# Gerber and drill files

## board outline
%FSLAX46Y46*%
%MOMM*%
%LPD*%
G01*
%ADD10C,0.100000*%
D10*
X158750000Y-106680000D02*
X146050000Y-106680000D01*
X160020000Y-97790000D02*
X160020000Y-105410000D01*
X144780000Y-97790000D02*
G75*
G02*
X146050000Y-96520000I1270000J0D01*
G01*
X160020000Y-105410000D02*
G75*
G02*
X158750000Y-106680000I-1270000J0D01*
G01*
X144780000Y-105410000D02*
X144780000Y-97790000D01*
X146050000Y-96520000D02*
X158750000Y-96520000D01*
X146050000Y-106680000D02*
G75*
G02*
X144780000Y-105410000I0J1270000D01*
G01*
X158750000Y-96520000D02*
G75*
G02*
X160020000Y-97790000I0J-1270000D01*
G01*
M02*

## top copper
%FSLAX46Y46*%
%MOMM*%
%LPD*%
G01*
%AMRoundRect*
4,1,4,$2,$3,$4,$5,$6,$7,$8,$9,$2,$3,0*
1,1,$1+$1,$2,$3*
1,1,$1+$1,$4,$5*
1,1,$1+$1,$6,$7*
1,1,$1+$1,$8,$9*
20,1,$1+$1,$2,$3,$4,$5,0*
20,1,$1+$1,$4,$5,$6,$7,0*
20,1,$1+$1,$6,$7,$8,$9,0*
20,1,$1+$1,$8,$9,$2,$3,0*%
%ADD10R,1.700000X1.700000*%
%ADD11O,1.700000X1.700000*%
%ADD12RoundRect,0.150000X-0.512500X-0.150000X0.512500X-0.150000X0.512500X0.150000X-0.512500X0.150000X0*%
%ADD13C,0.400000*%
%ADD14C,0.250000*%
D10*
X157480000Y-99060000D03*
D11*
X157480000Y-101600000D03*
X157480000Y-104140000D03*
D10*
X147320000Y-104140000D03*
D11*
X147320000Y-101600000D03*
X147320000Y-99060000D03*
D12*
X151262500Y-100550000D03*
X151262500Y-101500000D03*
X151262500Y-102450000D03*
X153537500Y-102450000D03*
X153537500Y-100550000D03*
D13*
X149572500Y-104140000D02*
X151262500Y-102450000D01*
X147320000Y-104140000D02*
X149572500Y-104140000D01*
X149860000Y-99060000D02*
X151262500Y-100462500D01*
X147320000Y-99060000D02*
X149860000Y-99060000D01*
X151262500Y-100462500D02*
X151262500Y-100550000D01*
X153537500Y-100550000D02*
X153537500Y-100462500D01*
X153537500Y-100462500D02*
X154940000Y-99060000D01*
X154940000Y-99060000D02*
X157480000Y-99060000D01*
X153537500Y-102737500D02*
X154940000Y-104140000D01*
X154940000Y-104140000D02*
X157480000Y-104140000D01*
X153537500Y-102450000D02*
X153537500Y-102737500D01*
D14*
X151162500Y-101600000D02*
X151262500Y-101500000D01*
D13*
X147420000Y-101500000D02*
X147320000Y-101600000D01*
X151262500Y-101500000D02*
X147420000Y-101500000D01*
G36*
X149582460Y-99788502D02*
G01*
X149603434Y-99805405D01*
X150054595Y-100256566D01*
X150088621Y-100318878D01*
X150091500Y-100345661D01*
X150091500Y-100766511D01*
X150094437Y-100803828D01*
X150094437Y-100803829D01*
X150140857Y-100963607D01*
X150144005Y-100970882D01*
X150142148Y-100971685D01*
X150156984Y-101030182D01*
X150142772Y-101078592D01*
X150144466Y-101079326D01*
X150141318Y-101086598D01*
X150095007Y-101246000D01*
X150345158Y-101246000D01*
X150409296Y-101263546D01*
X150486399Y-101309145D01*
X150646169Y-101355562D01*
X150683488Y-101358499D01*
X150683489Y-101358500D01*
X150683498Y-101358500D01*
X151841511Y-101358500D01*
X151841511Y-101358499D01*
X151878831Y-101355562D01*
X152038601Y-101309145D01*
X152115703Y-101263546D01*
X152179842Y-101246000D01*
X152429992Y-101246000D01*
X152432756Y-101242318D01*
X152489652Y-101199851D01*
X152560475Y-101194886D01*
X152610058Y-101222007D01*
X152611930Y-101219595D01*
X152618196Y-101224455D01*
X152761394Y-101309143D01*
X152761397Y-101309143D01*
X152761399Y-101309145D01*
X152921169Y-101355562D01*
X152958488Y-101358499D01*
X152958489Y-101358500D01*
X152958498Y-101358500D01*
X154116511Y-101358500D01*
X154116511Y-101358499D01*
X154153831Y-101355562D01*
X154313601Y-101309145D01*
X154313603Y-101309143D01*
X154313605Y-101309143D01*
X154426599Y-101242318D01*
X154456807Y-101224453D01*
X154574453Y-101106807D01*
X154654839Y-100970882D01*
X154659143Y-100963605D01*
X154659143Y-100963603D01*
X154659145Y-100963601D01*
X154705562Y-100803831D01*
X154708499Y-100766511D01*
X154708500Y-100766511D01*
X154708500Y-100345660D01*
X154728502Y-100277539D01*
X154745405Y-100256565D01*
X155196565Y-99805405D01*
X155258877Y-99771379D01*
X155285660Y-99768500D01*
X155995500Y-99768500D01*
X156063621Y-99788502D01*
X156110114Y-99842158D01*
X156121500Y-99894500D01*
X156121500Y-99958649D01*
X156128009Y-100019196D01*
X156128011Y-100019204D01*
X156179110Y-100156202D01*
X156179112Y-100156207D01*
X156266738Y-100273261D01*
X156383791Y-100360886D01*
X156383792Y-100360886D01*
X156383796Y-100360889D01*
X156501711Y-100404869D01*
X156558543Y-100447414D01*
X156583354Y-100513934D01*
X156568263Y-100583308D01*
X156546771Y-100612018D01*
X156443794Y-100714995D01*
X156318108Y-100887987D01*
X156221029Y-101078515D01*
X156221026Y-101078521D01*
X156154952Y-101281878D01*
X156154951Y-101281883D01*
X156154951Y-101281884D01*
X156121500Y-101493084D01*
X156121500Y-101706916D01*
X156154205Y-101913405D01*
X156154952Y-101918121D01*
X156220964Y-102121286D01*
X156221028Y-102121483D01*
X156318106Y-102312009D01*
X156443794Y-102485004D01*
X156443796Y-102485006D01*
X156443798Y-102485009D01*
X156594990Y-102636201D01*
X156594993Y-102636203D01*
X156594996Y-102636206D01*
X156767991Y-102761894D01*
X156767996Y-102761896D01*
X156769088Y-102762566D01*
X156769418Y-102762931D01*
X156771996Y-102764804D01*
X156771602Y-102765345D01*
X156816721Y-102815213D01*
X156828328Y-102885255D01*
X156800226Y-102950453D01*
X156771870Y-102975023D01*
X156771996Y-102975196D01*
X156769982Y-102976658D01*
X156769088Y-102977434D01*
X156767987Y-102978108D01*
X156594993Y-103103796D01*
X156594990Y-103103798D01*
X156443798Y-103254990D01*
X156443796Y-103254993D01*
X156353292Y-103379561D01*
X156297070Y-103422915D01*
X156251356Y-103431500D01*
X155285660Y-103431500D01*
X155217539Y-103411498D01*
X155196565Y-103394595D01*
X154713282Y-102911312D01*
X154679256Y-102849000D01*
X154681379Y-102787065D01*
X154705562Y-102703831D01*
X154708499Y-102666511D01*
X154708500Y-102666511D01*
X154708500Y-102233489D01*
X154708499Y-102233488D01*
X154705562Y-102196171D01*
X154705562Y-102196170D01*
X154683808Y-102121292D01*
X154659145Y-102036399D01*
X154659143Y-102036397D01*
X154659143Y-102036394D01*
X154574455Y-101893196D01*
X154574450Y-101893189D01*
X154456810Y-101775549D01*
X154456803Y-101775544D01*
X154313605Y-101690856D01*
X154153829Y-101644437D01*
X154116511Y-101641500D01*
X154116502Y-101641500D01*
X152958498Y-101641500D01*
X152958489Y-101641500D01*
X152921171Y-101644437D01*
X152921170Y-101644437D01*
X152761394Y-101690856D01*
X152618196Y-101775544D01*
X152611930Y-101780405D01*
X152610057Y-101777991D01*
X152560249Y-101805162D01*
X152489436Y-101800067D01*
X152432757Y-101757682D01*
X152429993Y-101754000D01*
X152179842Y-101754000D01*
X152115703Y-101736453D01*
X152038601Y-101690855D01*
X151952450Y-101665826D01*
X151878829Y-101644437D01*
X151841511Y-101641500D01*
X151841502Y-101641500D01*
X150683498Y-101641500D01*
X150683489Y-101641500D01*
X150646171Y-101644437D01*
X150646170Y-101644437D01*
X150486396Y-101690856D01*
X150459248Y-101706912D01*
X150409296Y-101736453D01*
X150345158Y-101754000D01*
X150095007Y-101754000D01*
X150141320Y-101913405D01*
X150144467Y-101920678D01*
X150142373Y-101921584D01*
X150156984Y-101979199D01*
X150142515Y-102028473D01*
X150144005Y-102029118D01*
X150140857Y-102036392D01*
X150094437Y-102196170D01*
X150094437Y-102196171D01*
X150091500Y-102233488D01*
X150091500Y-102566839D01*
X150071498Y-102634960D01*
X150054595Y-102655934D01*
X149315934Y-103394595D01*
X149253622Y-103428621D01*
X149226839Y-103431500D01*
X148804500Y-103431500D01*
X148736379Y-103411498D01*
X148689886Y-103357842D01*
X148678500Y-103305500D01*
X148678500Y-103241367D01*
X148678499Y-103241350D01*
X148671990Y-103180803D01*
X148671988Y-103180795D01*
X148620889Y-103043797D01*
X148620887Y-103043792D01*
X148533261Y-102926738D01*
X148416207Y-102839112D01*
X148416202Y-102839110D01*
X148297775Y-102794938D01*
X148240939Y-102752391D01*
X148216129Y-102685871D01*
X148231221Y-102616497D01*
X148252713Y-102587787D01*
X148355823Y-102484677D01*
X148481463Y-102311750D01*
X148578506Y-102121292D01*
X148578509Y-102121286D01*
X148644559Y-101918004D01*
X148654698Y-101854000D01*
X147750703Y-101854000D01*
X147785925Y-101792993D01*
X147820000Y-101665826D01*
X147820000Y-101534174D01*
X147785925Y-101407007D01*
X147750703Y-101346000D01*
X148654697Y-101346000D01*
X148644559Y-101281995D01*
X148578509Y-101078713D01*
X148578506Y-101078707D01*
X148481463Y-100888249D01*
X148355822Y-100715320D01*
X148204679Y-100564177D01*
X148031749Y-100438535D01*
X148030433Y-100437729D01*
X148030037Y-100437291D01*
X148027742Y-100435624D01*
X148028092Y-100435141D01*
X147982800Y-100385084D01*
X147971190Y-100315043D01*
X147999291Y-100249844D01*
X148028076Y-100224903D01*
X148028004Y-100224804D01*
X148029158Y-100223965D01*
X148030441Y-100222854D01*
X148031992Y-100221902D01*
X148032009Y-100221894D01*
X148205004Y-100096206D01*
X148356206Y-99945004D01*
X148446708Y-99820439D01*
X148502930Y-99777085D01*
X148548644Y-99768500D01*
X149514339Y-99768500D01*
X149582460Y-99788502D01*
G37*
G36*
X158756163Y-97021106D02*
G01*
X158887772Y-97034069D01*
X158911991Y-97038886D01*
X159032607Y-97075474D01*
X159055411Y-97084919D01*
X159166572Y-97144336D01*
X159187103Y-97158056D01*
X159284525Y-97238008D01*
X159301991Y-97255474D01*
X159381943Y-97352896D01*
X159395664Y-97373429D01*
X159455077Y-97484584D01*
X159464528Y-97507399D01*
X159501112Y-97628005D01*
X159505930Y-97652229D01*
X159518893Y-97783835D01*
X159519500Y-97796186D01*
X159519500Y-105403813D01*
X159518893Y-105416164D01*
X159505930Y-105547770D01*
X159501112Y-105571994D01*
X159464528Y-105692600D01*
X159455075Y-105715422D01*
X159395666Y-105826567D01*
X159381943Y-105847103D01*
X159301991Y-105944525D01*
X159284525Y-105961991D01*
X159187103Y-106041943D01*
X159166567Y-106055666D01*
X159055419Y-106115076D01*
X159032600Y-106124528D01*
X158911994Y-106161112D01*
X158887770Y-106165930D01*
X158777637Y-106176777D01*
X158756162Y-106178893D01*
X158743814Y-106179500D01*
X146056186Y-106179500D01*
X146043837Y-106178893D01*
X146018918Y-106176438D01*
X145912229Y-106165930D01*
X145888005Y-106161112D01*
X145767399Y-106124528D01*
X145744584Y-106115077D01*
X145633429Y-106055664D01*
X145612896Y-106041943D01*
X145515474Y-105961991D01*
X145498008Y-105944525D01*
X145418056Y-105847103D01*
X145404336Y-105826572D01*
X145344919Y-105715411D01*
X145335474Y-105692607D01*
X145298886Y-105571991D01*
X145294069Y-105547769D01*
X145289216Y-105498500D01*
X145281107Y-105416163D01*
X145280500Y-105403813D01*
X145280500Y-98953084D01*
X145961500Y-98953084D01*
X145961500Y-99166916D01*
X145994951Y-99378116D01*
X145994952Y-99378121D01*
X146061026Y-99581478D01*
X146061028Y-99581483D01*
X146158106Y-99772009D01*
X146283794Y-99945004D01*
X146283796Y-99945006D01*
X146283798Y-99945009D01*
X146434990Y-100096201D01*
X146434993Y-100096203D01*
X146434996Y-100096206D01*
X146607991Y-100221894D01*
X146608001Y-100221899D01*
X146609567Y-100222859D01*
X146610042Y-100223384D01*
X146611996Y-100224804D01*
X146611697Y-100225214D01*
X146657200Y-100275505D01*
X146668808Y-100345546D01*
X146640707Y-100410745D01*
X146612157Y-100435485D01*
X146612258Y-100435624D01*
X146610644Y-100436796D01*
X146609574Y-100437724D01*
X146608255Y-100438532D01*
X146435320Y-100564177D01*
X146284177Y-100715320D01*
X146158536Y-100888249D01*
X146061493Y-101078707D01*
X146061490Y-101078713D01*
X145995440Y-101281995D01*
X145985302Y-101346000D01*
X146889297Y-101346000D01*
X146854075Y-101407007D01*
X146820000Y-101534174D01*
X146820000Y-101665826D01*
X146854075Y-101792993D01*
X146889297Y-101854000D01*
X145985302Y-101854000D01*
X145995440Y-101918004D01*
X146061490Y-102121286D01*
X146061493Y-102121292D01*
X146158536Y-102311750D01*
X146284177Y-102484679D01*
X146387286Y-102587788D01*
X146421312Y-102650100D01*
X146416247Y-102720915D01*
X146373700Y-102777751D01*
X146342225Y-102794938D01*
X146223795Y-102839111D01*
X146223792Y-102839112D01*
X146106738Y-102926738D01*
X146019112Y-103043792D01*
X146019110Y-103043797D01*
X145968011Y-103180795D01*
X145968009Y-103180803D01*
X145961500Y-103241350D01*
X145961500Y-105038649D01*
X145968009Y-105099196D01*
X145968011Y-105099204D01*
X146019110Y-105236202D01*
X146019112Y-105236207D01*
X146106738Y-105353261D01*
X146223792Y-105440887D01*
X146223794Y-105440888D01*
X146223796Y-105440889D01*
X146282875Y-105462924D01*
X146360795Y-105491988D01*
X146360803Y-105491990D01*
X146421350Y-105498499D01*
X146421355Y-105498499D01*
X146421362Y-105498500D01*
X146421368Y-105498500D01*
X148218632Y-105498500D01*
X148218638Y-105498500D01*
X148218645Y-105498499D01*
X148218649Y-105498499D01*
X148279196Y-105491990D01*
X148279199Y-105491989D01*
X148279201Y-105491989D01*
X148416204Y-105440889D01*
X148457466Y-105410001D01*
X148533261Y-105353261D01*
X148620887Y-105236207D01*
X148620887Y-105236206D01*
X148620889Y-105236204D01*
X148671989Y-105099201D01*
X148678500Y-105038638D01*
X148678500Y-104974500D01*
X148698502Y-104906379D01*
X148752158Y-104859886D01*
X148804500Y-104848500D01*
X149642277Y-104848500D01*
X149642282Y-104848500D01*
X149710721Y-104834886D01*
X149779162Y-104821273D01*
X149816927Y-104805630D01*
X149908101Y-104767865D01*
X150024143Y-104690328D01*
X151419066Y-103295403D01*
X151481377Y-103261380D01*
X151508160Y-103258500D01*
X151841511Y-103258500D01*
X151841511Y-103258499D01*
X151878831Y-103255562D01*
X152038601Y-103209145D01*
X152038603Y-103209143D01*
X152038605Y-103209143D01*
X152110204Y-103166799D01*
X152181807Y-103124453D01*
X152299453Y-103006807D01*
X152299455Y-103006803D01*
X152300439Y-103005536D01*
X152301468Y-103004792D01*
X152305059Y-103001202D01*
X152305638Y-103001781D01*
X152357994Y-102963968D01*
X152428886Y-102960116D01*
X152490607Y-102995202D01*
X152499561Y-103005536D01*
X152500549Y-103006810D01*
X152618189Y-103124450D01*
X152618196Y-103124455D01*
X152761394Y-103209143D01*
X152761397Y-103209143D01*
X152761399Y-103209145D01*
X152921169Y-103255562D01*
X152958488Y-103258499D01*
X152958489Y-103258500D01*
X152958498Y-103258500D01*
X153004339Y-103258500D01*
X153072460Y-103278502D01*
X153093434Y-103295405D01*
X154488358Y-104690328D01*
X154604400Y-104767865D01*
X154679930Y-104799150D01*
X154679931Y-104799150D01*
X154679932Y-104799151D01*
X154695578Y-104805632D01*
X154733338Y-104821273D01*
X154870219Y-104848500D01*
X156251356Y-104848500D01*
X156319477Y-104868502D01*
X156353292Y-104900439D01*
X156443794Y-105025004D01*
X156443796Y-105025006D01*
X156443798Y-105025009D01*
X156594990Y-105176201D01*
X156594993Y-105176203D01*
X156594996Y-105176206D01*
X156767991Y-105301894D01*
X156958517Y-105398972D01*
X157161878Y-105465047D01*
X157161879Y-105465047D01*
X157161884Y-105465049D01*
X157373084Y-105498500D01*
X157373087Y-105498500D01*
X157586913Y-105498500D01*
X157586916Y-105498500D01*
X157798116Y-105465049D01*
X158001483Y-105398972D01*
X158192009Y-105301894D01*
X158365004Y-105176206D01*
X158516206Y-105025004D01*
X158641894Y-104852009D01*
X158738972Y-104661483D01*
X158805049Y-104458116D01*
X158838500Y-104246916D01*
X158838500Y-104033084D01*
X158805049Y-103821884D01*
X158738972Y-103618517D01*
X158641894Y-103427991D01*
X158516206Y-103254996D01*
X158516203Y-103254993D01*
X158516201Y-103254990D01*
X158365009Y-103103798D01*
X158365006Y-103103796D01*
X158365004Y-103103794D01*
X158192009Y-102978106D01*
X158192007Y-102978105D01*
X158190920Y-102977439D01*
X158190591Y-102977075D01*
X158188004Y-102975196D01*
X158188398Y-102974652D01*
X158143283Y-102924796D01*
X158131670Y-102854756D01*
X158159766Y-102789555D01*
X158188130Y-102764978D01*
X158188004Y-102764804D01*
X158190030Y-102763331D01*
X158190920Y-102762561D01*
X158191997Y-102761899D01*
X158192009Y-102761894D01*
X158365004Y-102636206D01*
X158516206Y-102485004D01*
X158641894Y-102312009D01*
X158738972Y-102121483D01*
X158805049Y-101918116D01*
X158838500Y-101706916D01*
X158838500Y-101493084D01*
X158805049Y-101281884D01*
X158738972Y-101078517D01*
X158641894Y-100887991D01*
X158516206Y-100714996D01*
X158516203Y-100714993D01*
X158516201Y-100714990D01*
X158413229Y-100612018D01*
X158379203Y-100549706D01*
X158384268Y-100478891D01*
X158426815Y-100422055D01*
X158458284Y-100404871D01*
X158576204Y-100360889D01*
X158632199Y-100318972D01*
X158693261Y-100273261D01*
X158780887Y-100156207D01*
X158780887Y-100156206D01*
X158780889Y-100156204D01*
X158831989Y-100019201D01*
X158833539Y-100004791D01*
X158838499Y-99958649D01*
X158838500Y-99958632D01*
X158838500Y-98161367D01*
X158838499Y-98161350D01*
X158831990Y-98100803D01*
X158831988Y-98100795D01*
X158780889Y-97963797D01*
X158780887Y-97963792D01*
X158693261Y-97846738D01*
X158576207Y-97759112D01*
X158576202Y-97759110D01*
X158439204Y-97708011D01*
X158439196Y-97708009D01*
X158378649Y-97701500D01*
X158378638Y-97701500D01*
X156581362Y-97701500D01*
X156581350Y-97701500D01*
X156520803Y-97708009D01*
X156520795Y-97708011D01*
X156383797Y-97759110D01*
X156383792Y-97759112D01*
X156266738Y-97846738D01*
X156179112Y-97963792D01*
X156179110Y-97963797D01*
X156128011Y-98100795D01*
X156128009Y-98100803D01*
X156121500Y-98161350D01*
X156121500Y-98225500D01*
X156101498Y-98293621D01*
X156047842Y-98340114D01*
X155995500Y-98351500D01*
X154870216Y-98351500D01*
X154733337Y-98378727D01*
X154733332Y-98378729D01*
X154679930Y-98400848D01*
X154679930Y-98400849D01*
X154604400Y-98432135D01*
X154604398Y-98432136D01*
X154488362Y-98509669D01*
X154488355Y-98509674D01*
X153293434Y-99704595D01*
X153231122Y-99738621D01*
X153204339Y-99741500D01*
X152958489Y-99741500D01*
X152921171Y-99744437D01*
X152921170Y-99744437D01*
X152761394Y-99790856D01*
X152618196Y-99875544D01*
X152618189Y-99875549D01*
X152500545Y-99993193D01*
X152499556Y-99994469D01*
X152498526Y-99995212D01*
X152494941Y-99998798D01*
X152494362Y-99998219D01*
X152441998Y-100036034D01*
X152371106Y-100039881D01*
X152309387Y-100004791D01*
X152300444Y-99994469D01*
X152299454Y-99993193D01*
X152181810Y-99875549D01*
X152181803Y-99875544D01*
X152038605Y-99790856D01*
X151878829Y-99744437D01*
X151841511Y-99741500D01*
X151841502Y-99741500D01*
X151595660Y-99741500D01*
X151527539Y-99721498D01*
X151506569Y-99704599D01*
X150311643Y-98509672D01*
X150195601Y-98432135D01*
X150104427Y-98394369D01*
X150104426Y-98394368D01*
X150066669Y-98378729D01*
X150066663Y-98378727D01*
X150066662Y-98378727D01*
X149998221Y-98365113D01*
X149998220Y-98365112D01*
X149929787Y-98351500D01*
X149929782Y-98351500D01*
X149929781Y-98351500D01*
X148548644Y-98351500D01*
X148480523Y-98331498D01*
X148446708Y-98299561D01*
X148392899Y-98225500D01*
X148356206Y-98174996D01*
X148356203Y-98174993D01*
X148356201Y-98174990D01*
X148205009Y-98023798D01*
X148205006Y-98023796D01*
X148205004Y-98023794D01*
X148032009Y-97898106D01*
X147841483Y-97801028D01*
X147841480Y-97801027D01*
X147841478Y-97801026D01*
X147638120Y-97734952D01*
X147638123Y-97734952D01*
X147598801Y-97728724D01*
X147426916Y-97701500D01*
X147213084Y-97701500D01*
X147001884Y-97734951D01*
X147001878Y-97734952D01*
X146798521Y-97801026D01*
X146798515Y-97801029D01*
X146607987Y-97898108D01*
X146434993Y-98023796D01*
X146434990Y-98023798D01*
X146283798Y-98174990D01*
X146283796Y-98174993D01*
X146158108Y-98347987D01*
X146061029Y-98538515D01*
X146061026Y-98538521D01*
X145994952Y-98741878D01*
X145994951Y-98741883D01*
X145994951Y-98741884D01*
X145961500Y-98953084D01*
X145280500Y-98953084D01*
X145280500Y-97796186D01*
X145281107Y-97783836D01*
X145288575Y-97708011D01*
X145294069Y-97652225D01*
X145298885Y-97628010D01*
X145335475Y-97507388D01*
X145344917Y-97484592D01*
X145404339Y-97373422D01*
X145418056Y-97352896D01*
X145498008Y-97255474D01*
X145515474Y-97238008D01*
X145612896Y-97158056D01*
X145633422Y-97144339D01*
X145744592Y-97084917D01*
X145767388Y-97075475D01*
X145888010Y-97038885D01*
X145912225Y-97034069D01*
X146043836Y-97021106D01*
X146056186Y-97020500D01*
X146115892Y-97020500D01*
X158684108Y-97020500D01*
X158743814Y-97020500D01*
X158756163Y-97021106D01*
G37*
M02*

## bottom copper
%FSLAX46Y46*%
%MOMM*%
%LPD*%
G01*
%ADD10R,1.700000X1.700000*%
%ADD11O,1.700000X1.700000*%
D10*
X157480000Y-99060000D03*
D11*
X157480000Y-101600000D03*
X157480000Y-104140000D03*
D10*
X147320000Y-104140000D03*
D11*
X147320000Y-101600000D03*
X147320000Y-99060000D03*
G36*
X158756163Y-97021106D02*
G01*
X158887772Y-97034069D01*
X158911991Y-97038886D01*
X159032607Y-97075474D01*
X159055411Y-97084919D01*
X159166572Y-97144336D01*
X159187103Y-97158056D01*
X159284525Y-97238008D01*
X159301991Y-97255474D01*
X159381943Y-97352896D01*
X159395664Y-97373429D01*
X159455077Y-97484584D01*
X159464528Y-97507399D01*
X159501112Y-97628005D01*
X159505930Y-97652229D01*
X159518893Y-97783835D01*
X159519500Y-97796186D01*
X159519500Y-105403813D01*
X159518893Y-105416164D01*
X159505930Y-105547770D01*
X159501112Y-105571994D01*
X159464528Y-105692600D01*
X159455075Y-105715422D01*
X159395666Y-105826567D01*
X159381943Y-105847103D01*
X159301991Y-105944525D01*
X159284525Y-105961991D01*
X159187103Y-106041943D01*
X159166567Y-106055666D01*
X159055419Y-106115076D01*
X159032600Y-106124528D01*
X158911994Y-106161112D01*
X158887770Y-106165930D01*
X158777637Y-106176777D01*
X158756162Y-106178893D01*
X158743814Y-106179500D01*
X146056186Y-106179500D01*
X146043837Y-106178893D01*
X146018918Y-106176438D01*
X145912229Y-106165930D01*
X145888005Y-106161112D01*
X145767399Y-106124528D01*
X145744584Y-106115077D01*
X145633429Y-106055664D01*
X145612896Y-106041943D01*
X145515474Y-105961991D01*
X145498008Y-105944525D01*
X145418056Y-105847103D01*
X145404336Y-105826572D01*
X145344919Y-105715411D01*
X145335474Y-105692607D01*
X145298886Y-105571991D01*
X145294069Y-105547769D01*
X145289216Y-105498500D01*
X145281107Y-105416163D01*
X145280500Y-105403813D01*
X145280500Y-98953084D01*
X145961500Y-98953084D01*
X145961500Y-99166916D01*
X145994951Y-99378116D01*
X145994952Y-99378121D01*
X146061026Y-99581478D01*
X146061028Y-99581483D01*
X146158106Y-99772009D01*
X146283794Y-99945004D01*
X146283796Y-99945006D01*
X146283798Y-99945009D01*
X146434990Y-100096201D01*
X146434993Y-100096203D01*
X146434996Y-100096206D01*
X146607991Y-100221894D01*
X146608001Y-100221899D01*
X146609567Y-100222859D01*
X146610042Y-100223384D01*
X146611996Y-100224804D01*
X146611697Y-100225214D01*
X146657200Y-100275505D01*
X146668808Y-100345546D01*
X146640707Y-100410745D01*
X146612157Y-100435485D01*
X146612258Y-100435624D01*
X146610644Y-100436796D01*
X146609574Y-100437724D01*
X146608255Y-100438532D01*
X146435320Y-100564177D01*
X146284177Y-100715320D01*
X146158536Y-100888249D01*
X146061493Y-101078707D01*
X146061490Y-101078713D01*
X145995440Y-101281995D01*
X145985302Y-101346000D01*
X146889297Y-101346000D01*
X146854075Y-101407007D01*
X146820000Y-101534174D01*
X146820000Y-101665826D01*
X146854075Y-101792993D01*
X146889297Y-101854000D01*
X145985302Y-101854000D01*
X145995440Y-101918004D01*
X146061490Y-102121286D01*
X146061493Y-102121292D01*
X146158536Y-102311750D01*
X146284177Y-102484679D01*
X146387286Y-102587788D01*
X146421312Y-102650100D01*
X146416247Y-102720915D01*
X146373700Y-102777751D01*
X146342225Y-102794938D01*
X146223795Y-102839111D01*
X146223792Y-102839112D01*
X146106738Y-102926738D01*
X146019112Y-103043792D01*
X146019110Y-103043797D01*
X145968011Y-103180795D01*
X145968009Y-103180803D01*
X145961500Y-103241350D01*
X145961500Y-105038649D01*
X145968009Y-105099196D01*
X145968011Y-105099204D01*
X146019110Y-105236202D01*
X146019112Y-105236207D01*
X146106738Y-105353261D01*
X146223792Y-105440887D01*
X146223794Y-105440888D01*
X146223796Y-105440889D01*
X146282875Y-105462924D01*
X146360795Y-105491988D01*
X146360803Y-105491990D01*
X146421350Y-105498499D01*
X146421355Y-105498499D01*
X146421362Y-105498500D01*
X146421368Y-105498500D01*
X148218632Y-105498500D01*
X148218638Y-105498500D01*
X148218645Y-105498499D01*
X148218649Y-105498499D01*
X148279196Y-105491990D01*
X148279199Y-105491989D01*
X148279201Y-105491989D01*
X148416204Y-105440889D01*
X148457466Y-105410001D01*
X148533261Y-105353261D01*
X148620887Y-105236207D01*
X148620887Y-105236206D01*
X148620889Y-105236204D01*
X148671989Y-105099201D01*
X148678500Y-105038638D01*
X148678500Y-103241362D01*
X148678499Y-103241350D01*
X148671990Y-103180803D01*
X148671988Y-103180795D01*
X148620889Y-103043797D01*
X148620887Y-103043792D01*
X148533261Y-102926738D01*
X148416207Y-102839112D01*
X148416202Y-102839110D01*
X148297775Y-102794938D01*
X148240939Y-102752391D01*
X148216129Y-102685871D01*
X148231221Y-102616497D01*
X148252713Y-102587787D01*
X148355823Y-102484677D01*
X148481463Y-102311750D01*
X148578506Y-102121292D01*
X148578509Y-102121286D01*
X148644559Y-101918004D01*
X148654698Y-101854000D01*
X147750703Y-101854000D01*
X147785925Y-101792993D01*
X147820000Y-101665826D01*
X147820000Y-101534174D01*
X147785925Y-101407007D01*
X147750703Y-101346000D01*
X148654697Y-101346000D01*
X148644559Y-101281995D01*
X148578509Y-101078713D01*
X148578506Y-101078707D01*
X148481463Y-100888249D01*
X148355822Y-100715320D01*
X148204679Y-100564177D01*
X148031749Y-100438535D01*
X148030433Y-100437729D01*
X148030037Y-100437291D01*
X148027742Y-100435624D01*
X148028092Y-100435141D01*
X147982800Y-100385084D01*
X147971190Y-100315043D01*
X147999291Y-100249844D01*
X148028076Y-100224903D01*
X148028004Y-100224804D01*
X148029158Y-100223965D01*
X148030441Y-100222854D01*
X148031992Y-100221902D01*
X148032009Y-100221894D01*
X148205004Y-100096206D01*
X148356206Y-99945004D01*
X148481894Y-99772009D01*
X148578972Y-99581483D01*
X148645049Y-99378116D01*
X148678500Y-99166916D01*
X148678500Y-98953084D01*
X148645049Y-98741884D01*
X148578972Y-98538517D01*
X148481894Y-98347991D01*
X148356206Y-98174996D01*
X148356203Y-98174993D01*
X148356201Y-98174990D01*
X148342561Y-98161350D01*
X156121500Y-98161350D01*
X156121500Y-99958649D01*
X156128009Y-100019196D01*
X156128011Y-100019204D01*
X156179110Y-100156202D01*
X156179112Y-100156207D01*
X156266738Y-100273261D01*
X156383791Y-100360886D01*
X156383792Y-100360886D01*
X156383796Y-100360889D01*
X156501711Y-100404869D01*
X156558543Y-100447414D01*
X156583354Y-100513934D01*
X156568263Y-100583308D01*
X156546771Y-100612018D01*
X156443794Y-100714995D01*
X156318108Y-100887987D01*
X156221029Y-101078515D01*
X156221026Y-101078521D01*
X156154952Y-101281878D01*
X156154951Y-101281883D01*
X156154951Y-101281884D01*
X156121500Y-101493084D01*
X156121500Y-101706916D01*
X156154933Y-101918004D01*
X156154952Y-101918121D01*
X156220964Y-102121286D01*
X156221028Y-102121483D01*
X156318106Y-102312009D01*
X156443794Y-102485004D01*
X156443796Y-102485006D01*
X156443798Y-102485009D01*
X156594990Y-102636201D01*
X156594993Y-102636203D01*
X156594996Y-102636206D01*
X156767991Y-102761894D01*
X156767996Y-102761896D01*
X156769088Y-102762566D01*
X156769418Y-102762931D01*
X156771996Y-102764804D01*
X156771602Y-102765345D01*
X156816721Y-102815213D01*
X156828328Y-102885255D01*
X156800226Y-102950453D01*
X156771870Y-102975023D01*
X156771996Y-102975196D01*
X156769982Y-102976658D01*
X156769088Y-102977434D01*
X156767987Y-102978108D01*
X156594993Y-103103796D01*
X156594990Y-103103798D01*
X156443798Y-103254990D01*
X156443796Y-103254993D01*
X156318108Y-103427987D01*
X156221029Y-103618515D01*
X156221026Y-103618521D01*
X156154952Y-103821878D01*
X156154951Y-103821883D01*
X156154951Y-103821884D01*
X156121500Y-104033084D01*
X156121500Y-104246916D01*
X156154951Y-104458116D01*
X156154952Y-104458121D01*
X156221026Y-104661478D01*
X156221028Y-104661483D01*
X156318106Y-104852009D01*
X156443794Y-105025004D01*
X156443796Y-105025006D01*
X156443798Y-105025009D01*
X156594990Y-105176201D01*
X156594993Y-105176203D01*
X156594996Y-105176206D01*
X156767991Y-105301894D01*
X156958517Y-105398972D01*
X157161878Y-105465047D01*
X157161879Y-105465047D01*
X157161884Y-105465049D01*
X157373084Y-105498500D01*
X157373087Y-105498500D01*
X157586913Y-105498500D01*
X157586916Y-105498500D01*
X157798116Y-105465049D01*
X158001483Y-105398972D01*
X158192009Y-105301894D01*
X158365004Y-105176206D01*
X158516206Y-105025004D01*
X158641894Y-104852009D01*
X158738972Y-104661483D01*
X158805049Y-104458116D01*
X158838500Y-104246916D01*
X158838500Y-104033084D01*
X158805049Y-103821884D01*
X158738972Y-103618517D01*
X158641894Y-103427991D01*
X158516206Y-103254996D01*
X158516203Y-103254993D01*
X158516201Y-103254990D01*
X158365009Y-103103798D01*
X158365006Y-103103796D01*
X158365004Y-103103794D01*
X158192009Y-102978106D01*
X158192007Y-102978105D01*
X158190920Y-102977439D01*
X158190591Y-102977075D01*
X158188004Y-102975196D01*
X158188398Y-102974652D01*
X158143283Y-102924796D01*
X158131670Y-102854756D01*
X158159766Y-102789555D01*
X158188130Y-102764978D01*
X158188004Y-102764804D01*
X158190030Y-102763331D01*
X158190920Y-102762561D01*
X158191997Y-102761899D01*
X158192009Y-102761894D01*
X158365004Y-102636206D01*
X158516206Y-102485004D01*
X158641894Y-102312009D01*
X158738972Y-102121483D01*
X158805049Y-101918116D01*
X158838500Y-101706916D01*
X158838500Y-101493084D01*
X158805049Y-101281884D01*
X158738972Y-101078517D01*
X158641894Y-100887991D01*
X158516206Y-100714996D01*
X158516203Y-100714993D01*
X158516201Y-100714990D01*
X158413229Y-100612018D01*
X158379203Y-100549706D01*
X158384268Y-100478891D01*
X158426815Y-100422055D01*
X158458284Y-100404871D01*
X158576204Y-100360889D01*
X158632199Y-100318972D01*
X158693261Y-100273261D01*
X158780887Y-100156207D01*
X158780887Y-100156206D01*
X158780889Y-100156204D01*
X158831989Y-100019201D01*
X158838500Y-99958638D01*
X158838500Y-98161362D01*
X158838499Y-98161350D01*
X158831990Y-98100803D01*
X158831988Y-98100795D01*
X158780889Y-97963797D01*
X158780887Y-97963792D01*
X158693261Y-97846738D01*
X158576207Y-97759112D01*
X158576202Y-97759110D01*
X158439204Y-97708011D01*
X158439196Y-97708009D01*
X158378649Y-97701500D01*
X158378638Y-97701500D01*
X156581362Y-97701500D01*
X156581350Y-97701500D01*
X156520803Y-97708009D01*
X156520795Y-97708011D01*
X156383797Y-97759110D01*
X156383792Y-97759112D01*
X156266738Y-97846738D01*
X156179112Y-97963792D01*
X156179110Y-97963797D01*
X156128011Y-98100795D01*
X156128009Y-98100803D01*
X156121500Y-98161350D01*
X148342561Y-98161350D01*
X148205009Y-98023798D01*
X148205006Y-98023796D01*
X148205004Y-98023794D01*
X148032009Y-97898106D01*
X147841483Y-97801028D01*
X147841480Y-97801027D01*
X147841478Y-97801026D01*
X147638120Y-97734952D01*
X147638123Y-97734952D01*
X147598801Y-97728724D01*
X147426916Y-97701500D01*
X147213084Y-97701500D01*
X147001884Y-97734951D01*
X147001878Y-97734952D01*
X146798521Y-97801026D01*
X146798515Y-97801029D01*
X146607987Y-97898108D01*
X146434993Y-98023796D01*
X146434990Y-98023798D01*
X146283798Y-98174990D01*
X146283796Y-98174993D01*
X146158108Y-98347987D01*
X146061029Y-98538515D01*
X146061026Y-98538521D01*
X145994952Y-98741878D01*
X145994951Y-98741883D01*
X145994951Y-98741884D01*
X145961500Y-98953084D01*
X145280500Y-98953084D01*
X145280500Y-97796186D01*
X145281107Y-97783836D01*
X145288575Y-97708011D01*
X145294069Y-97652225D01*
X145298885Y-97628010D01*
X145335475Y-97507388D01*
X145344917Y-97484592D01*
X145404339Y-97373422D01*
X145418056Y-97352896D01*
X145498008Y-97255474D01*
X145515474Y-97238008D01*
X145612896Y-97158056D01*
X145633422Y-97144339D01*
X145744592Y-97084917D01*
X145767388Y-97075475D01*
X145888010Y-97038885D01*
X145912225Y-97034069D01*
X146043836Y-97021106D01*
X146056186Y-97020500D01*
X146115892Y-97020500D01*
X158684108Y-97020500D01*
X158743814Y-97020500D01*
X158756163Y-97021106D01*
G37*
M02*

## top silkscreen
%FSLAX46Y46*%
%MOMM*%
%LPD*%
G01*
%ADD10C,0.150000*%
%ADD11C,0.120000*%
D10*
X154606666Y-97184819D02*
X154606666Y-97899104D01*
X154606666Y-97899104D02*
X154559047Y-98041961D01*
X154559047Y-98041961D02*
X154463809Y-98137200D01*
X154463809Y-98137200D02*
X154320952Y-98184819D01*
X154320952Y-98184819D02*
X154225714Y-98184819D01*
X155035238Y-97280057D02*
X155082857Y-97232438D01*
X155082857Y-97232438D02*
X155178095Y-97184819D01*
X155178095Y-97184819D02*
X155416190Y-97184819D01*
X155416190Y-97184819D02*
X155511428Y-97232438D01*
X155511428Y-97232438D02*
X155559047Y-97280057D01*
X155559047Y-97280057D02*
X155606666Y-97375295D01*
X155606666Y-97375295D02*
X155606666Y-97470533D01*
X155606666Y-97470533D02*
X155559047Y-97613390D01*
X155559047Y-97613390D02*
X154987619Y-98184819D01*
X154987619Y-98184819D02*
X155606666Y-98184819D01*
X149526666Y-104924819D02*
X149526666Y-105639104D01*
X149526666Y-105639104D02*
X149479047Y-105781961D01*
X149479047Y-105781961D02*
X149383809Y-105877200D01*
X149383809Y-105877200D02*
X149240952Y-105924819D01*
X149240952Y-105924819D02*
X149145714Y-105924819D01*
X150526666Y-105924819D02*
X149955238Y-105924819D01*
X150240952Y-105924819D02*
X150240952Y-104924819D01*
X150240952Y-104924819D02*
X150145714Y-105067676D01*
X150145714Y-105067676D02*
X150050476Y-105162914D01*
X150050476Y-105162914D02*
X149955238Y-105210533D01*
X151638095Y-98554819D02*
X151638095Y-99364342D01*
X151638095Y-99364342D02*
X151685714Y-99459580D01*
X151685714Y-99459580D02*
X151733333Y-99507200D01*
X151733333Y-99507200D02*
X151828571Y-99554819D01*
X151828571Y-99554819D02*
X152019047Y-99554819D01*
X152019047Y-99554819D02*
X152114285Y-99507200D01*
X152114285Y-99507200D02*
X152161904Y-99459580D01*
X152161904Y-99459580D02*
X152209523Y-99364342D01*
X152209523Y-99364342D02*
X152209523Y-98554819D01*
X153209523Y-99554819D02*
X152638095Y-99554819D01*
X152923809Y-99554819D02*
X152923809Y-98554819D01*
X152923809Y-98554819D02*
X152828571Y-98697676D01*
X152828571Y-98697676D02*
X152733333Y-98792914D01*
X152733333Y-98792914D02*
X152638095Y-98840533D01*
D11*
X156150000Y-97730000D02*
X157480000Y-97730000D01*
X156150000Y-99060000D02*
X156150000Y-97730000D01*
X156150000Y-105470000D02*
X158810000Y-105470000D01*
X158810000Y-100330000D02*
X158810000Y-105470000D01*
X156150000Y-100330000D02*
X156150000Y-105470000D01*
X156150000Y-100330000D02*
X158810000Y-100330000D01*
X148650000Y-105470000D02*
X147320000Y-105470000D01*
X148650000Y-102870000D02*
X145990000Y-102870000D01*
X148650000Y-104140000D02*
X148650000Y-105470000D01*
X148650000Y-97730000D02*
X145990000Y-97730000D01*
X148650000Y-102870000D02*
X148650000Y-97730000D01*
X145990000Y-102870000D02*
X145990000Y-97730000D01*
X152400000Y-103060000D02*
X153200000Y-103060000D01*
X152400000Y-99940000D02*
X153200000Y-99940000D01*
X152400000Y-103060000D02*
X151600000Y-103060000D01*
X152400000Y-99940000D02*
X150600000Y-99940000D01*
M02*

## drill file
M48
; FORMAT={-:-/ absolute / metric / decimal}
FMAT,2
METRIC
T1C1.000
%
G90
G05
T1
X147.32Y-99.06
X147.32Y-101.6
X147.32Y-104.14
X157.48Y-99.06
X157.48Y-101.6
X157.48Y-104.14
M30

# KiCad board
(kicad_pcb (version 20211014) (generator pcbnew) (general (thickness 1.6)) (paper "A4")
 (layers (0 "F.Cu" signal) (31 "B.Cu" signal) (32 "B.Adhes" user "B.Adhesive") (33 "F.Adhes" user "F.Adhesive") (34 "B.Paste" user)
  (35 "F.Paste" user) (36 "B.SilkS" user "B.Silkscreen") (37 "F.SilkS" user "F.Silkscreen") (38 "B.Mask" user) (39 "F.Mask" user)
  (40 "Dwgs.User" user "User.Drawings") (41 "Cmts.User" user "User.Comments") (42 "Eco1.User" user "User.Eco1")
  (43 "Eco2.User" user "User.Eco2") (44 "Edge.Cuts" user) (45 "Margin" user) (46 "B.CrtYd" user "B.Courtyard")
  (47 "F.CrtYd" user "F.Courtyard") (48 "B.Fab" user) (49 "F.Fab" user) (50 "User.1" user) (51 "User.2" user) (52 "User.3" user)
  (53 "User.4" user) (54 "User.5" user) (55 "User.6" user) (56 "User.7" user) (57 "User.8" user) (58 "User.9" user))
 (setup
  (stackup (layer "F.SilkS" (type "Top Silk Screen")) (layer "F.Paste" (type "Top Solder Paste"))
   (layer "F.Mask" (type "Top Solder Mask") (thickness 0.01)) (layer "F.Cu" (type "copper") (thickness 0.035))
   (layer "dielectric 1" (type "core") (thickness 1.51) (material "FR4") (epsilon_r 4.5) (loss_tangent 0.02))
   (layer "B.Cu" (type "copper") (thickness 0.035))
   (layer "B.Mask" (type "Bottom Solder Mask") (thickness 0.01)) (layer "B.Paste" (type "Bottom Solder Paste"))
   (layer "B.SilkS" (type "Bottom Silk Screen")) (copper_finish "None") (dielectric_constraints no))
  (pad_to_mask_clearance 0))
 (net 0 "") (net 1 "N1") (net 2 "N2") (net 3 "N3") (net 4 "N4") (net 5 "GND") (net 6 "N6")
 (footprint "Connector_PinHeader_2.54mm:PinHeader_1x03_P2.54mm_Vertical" (layer "F.Cu") (at 157.48 99.06)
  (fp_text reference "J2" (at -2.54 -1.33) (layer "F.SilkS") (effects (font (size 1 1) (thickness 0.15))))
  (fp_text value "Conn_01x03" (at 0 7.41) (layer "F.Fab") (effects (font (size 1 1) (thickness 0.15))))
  (fp_line (start -1.33 -1.33) (end 0 -1.33) (layer "F.SilkS") (width 0.12))
  (fp_line (start -1.33 0) (end -1.33 -1.33) (layer "F.SilkS") (width 0.12))
  (fp_line (start -1.33 6.41) (end 1.33 6.41) (layer "F.SilkS") (width 0.12))
  (fp_line (start 1.33 1.27) (end 1.33 6.41) (layer "F.SilkS") (width 0.12))
  (fp_line (start -1.33 1.27) (end -1.33 6.41) (layer "F.SilkS") (width 0.12))
  (fp_line (start -1.33 1.27) (end 1.33 1.27) (layer "F.SilkS") (width 0.12))
  (pad "1" thru_hole rect (at 0 0) (size 1.7 1.7) (drill 1) (layers *.Cu *.Mask) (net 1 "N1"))
  (pad "2" thru_hole oval (at 0 2.54) (size 1.7 1.7) (drill 1) (layers *.Cu *.Mask) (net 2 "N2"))
  (pad "3" thru_hole oval (at 0 5.08) (size 1.7 1.7) (drill 1) (layers *.Cu *.Mask) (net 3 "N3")))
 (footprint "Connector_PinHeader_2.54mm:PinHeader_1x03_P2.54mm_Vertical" (layer "F.Cu") (at 147.32 104.14 180)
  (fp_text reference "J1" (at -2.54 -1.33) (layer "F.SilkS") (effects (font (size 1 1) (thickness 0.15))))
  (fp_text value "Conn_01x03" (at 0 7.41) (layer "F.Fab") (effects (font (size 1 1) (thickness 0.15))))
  (fp_line (start -1.33 -1.33) (end 0 -1.33) (layer "F.SilkS") (width 0.12))
  (fp_line (start -1.33 1.27) (end 1.33 1.27) (layer "F.SilkS") (width 0.12))
  (fp_line (start -1.33 0) (end -1.33 -1.33) (layer "F.SilkS") (width 0.12))
  (fp_line (start -1.33 6.41) (end 1.33 6.41) (layer "F.SilkS") (width 0.12))
  (fp_line (start -1.33 1.27) (end -1.33 6.41) (layer "F.SilkS") (width 0.12))
  (fp_line (start 1.33 1.27) (end 1.33 6.41) (layer "F.SilkS") (width 0.12))
  (pad "1" thru_hole rect (at 0 0 180) (size 1.7 1.7) (drill 1) (layers *.Cu *.Mask) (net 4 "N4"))
  (pad "2" thru_hole oval (at 0 2.54 180) (size 1.7 1.7) (drill 1) (layers *.Cu *.Mask) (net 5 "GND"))
  (pad "3" thru_hole oval (at 0 5.08 180) (size 1.7 1.7) (drill 1) (layers *.Cu *.Mask) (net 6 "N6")))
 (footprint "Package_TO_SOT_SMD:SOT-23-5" (layer "F.Cu") (at 152.4 101.5)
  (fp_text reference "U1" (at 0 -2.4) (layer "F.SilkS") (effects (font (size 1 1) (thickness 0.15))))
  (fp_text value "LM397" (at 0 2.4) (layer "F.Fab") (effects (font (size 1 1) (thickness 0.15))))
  (fp_line (start 0 1.56) (end 0.8 1.56) (layer "F.SilkS") (width 0.12))
  (fp_line (start 0 -1.56) (end 0.8 -1.56) (layer "F.SilkS") (width 0.12))
  (fp_line (start 0 1.56) (end -0.8 1.56) (layer "F.SilkS") (width 0.12))
  (fp_line (start 0 -1.56) (end -1.8 -1.56) (layer "F.SilkS") (width 0.12))
  (pad "1" smd roundrect (at -1.1375 -0.95) (size 1.325 0.6) (layers "F.Cu" "F.Paste" "F.Mask") (roundrect_rratio 0.25) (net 6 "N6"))
  (pad "2" smd roundrect (at -1.1375 0) (size 1.325 0.6) (layers "F.Cu" "F.Paste" "F.Mask") (roundrect_rratio 0.25) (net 5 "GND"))
  (pad "3" smd roundrect (at -1.1375 0.95) (size 1.325 0.6) (layers "F.Cu" "F.Paste" "F.Mask") (roundrect_rratio 0.25) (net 4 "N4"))
  (pad "4" smd roundrect (at 1.1375 0.95) (size 1.325 0.6) (layers "F.Cu" "F.Paste" "F.Mask") (roundrect_rratio 0.25) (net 3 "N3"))
  (pad "5" smd roundrect (at 1.1375 -0.95) (size 1.325 0.6) (layers "F.Cu" "F.Paste" "F.Mask") (roundrect_rratio 0.25) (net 1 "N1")))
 (gr_line (start 158.75 106.68) (end 146.05 106.68) (layer "Edge.Cuts") (width 0.1))
 (gr_line (start 160.02 97.79) (end 160.02 105.41) (layer "Edge.Cuts") (width 0.1))
 (gr_arc (start 144.78 97.79) (mid 145.151974 96.891974) (end 146.05 96.52) (layer "Edge.Cuts") (width 0.1))
 (gr_arc (start 160.02 105.41) (mid 159.648026 106.308026) (end 158.75 106.68) (layer "Edge.Cuts") (width 0.1))
 (gr_line (start 144.78 105.41) (end 144.78 97.79) (layer "Edge.Cuts") (width 0.1))
 (gr_line (start 146.05 96.52) (end 158.75 96.52) (layer "Edge.Cuts") (width 0.1))
 (gr_arc (start 146.05 106.68) (mid 145.151974 106.308026) (end 144.78 105.41) (layer "Edge.Cuts") (width 0.1))
 (gr_arc (start 158.75 96.52) (mid 159.648026 96.891974) (end 160.02 97.79) (layer "Edge.Cuts") (width 0.1))
 (segment (start 149.5725 104.14) (end 151.2625 102.45) (width 0.4) (layer "F.Cu") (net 4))
 (segment (start 147.32 104.14) (end 149.5725 104.14) (width 0.4) (layer "F.Cu") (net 4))
 (segment (start 149.86 99.06) (end 151.2625 100.4625) (width 0.4) (layer "F.Cu") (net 6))
 (segment (start 147.32 99.06) (end 149.86 99.06) (width 0.4) (layer "F.Cu") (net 6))
 (segment (start 151.2625 100.4625) (end 151.2625 100.55) (width 0.4) (layer "F.Cu") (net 6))
 (segment (start 153.5375 100.55) (end 153.5375 100.4625) (width 0.4) (layer "F.Cu") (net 1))
 (segment (start 153.5375 100.4625) (end 154.94 99.06) (width 0.4) (layer "F.Cu") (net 1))
 (segment (start 154.94 99.06) (end 157.48 99.06) (width 0.4) (layer "F.Cu") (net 1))
 (segment (start 153.5375 102.7375) (end 154.94 104.14) (width 0.4) (layer "F.Cu") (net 3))
 (segment (start 154.94 104.14) (end 157.48 104.14) (width 0.4) (layer "F.Cu") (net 3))
 (segment (start 153.5375 102.45) (end 153.5375 102.7375) (width 0.4) (layer "F.Cu") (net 3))
 (segment (start 151.1625 101.6) (end 151.2625 101.5) (width 0.25) (layer "F.Cu") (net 5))
 (segment (start 147.42 101.5) (end 147.32 101.6) (width 0.4) (layer "F.Cu") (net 5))
 (segment (start 151.2625 101.5) (end 147.42 101.5) (width 0.4) (layer "F.Cu") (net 5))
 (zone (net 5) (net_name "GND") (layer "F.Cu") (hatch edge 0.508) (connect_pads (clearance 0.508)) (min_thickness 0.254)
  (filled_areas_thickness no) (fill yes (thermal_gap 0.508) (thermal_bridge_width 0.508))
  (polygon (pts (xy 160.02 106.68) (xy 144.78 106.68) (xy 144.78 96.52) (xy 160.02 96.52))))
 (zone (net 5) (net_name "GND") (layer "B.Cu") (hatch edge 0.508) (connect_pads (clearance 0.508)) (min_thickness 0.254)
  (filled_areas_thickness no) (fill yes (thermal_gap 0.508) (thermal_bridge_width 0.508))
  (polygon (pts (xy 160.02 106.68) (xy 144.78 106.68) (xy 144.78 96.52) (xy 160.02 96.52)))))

